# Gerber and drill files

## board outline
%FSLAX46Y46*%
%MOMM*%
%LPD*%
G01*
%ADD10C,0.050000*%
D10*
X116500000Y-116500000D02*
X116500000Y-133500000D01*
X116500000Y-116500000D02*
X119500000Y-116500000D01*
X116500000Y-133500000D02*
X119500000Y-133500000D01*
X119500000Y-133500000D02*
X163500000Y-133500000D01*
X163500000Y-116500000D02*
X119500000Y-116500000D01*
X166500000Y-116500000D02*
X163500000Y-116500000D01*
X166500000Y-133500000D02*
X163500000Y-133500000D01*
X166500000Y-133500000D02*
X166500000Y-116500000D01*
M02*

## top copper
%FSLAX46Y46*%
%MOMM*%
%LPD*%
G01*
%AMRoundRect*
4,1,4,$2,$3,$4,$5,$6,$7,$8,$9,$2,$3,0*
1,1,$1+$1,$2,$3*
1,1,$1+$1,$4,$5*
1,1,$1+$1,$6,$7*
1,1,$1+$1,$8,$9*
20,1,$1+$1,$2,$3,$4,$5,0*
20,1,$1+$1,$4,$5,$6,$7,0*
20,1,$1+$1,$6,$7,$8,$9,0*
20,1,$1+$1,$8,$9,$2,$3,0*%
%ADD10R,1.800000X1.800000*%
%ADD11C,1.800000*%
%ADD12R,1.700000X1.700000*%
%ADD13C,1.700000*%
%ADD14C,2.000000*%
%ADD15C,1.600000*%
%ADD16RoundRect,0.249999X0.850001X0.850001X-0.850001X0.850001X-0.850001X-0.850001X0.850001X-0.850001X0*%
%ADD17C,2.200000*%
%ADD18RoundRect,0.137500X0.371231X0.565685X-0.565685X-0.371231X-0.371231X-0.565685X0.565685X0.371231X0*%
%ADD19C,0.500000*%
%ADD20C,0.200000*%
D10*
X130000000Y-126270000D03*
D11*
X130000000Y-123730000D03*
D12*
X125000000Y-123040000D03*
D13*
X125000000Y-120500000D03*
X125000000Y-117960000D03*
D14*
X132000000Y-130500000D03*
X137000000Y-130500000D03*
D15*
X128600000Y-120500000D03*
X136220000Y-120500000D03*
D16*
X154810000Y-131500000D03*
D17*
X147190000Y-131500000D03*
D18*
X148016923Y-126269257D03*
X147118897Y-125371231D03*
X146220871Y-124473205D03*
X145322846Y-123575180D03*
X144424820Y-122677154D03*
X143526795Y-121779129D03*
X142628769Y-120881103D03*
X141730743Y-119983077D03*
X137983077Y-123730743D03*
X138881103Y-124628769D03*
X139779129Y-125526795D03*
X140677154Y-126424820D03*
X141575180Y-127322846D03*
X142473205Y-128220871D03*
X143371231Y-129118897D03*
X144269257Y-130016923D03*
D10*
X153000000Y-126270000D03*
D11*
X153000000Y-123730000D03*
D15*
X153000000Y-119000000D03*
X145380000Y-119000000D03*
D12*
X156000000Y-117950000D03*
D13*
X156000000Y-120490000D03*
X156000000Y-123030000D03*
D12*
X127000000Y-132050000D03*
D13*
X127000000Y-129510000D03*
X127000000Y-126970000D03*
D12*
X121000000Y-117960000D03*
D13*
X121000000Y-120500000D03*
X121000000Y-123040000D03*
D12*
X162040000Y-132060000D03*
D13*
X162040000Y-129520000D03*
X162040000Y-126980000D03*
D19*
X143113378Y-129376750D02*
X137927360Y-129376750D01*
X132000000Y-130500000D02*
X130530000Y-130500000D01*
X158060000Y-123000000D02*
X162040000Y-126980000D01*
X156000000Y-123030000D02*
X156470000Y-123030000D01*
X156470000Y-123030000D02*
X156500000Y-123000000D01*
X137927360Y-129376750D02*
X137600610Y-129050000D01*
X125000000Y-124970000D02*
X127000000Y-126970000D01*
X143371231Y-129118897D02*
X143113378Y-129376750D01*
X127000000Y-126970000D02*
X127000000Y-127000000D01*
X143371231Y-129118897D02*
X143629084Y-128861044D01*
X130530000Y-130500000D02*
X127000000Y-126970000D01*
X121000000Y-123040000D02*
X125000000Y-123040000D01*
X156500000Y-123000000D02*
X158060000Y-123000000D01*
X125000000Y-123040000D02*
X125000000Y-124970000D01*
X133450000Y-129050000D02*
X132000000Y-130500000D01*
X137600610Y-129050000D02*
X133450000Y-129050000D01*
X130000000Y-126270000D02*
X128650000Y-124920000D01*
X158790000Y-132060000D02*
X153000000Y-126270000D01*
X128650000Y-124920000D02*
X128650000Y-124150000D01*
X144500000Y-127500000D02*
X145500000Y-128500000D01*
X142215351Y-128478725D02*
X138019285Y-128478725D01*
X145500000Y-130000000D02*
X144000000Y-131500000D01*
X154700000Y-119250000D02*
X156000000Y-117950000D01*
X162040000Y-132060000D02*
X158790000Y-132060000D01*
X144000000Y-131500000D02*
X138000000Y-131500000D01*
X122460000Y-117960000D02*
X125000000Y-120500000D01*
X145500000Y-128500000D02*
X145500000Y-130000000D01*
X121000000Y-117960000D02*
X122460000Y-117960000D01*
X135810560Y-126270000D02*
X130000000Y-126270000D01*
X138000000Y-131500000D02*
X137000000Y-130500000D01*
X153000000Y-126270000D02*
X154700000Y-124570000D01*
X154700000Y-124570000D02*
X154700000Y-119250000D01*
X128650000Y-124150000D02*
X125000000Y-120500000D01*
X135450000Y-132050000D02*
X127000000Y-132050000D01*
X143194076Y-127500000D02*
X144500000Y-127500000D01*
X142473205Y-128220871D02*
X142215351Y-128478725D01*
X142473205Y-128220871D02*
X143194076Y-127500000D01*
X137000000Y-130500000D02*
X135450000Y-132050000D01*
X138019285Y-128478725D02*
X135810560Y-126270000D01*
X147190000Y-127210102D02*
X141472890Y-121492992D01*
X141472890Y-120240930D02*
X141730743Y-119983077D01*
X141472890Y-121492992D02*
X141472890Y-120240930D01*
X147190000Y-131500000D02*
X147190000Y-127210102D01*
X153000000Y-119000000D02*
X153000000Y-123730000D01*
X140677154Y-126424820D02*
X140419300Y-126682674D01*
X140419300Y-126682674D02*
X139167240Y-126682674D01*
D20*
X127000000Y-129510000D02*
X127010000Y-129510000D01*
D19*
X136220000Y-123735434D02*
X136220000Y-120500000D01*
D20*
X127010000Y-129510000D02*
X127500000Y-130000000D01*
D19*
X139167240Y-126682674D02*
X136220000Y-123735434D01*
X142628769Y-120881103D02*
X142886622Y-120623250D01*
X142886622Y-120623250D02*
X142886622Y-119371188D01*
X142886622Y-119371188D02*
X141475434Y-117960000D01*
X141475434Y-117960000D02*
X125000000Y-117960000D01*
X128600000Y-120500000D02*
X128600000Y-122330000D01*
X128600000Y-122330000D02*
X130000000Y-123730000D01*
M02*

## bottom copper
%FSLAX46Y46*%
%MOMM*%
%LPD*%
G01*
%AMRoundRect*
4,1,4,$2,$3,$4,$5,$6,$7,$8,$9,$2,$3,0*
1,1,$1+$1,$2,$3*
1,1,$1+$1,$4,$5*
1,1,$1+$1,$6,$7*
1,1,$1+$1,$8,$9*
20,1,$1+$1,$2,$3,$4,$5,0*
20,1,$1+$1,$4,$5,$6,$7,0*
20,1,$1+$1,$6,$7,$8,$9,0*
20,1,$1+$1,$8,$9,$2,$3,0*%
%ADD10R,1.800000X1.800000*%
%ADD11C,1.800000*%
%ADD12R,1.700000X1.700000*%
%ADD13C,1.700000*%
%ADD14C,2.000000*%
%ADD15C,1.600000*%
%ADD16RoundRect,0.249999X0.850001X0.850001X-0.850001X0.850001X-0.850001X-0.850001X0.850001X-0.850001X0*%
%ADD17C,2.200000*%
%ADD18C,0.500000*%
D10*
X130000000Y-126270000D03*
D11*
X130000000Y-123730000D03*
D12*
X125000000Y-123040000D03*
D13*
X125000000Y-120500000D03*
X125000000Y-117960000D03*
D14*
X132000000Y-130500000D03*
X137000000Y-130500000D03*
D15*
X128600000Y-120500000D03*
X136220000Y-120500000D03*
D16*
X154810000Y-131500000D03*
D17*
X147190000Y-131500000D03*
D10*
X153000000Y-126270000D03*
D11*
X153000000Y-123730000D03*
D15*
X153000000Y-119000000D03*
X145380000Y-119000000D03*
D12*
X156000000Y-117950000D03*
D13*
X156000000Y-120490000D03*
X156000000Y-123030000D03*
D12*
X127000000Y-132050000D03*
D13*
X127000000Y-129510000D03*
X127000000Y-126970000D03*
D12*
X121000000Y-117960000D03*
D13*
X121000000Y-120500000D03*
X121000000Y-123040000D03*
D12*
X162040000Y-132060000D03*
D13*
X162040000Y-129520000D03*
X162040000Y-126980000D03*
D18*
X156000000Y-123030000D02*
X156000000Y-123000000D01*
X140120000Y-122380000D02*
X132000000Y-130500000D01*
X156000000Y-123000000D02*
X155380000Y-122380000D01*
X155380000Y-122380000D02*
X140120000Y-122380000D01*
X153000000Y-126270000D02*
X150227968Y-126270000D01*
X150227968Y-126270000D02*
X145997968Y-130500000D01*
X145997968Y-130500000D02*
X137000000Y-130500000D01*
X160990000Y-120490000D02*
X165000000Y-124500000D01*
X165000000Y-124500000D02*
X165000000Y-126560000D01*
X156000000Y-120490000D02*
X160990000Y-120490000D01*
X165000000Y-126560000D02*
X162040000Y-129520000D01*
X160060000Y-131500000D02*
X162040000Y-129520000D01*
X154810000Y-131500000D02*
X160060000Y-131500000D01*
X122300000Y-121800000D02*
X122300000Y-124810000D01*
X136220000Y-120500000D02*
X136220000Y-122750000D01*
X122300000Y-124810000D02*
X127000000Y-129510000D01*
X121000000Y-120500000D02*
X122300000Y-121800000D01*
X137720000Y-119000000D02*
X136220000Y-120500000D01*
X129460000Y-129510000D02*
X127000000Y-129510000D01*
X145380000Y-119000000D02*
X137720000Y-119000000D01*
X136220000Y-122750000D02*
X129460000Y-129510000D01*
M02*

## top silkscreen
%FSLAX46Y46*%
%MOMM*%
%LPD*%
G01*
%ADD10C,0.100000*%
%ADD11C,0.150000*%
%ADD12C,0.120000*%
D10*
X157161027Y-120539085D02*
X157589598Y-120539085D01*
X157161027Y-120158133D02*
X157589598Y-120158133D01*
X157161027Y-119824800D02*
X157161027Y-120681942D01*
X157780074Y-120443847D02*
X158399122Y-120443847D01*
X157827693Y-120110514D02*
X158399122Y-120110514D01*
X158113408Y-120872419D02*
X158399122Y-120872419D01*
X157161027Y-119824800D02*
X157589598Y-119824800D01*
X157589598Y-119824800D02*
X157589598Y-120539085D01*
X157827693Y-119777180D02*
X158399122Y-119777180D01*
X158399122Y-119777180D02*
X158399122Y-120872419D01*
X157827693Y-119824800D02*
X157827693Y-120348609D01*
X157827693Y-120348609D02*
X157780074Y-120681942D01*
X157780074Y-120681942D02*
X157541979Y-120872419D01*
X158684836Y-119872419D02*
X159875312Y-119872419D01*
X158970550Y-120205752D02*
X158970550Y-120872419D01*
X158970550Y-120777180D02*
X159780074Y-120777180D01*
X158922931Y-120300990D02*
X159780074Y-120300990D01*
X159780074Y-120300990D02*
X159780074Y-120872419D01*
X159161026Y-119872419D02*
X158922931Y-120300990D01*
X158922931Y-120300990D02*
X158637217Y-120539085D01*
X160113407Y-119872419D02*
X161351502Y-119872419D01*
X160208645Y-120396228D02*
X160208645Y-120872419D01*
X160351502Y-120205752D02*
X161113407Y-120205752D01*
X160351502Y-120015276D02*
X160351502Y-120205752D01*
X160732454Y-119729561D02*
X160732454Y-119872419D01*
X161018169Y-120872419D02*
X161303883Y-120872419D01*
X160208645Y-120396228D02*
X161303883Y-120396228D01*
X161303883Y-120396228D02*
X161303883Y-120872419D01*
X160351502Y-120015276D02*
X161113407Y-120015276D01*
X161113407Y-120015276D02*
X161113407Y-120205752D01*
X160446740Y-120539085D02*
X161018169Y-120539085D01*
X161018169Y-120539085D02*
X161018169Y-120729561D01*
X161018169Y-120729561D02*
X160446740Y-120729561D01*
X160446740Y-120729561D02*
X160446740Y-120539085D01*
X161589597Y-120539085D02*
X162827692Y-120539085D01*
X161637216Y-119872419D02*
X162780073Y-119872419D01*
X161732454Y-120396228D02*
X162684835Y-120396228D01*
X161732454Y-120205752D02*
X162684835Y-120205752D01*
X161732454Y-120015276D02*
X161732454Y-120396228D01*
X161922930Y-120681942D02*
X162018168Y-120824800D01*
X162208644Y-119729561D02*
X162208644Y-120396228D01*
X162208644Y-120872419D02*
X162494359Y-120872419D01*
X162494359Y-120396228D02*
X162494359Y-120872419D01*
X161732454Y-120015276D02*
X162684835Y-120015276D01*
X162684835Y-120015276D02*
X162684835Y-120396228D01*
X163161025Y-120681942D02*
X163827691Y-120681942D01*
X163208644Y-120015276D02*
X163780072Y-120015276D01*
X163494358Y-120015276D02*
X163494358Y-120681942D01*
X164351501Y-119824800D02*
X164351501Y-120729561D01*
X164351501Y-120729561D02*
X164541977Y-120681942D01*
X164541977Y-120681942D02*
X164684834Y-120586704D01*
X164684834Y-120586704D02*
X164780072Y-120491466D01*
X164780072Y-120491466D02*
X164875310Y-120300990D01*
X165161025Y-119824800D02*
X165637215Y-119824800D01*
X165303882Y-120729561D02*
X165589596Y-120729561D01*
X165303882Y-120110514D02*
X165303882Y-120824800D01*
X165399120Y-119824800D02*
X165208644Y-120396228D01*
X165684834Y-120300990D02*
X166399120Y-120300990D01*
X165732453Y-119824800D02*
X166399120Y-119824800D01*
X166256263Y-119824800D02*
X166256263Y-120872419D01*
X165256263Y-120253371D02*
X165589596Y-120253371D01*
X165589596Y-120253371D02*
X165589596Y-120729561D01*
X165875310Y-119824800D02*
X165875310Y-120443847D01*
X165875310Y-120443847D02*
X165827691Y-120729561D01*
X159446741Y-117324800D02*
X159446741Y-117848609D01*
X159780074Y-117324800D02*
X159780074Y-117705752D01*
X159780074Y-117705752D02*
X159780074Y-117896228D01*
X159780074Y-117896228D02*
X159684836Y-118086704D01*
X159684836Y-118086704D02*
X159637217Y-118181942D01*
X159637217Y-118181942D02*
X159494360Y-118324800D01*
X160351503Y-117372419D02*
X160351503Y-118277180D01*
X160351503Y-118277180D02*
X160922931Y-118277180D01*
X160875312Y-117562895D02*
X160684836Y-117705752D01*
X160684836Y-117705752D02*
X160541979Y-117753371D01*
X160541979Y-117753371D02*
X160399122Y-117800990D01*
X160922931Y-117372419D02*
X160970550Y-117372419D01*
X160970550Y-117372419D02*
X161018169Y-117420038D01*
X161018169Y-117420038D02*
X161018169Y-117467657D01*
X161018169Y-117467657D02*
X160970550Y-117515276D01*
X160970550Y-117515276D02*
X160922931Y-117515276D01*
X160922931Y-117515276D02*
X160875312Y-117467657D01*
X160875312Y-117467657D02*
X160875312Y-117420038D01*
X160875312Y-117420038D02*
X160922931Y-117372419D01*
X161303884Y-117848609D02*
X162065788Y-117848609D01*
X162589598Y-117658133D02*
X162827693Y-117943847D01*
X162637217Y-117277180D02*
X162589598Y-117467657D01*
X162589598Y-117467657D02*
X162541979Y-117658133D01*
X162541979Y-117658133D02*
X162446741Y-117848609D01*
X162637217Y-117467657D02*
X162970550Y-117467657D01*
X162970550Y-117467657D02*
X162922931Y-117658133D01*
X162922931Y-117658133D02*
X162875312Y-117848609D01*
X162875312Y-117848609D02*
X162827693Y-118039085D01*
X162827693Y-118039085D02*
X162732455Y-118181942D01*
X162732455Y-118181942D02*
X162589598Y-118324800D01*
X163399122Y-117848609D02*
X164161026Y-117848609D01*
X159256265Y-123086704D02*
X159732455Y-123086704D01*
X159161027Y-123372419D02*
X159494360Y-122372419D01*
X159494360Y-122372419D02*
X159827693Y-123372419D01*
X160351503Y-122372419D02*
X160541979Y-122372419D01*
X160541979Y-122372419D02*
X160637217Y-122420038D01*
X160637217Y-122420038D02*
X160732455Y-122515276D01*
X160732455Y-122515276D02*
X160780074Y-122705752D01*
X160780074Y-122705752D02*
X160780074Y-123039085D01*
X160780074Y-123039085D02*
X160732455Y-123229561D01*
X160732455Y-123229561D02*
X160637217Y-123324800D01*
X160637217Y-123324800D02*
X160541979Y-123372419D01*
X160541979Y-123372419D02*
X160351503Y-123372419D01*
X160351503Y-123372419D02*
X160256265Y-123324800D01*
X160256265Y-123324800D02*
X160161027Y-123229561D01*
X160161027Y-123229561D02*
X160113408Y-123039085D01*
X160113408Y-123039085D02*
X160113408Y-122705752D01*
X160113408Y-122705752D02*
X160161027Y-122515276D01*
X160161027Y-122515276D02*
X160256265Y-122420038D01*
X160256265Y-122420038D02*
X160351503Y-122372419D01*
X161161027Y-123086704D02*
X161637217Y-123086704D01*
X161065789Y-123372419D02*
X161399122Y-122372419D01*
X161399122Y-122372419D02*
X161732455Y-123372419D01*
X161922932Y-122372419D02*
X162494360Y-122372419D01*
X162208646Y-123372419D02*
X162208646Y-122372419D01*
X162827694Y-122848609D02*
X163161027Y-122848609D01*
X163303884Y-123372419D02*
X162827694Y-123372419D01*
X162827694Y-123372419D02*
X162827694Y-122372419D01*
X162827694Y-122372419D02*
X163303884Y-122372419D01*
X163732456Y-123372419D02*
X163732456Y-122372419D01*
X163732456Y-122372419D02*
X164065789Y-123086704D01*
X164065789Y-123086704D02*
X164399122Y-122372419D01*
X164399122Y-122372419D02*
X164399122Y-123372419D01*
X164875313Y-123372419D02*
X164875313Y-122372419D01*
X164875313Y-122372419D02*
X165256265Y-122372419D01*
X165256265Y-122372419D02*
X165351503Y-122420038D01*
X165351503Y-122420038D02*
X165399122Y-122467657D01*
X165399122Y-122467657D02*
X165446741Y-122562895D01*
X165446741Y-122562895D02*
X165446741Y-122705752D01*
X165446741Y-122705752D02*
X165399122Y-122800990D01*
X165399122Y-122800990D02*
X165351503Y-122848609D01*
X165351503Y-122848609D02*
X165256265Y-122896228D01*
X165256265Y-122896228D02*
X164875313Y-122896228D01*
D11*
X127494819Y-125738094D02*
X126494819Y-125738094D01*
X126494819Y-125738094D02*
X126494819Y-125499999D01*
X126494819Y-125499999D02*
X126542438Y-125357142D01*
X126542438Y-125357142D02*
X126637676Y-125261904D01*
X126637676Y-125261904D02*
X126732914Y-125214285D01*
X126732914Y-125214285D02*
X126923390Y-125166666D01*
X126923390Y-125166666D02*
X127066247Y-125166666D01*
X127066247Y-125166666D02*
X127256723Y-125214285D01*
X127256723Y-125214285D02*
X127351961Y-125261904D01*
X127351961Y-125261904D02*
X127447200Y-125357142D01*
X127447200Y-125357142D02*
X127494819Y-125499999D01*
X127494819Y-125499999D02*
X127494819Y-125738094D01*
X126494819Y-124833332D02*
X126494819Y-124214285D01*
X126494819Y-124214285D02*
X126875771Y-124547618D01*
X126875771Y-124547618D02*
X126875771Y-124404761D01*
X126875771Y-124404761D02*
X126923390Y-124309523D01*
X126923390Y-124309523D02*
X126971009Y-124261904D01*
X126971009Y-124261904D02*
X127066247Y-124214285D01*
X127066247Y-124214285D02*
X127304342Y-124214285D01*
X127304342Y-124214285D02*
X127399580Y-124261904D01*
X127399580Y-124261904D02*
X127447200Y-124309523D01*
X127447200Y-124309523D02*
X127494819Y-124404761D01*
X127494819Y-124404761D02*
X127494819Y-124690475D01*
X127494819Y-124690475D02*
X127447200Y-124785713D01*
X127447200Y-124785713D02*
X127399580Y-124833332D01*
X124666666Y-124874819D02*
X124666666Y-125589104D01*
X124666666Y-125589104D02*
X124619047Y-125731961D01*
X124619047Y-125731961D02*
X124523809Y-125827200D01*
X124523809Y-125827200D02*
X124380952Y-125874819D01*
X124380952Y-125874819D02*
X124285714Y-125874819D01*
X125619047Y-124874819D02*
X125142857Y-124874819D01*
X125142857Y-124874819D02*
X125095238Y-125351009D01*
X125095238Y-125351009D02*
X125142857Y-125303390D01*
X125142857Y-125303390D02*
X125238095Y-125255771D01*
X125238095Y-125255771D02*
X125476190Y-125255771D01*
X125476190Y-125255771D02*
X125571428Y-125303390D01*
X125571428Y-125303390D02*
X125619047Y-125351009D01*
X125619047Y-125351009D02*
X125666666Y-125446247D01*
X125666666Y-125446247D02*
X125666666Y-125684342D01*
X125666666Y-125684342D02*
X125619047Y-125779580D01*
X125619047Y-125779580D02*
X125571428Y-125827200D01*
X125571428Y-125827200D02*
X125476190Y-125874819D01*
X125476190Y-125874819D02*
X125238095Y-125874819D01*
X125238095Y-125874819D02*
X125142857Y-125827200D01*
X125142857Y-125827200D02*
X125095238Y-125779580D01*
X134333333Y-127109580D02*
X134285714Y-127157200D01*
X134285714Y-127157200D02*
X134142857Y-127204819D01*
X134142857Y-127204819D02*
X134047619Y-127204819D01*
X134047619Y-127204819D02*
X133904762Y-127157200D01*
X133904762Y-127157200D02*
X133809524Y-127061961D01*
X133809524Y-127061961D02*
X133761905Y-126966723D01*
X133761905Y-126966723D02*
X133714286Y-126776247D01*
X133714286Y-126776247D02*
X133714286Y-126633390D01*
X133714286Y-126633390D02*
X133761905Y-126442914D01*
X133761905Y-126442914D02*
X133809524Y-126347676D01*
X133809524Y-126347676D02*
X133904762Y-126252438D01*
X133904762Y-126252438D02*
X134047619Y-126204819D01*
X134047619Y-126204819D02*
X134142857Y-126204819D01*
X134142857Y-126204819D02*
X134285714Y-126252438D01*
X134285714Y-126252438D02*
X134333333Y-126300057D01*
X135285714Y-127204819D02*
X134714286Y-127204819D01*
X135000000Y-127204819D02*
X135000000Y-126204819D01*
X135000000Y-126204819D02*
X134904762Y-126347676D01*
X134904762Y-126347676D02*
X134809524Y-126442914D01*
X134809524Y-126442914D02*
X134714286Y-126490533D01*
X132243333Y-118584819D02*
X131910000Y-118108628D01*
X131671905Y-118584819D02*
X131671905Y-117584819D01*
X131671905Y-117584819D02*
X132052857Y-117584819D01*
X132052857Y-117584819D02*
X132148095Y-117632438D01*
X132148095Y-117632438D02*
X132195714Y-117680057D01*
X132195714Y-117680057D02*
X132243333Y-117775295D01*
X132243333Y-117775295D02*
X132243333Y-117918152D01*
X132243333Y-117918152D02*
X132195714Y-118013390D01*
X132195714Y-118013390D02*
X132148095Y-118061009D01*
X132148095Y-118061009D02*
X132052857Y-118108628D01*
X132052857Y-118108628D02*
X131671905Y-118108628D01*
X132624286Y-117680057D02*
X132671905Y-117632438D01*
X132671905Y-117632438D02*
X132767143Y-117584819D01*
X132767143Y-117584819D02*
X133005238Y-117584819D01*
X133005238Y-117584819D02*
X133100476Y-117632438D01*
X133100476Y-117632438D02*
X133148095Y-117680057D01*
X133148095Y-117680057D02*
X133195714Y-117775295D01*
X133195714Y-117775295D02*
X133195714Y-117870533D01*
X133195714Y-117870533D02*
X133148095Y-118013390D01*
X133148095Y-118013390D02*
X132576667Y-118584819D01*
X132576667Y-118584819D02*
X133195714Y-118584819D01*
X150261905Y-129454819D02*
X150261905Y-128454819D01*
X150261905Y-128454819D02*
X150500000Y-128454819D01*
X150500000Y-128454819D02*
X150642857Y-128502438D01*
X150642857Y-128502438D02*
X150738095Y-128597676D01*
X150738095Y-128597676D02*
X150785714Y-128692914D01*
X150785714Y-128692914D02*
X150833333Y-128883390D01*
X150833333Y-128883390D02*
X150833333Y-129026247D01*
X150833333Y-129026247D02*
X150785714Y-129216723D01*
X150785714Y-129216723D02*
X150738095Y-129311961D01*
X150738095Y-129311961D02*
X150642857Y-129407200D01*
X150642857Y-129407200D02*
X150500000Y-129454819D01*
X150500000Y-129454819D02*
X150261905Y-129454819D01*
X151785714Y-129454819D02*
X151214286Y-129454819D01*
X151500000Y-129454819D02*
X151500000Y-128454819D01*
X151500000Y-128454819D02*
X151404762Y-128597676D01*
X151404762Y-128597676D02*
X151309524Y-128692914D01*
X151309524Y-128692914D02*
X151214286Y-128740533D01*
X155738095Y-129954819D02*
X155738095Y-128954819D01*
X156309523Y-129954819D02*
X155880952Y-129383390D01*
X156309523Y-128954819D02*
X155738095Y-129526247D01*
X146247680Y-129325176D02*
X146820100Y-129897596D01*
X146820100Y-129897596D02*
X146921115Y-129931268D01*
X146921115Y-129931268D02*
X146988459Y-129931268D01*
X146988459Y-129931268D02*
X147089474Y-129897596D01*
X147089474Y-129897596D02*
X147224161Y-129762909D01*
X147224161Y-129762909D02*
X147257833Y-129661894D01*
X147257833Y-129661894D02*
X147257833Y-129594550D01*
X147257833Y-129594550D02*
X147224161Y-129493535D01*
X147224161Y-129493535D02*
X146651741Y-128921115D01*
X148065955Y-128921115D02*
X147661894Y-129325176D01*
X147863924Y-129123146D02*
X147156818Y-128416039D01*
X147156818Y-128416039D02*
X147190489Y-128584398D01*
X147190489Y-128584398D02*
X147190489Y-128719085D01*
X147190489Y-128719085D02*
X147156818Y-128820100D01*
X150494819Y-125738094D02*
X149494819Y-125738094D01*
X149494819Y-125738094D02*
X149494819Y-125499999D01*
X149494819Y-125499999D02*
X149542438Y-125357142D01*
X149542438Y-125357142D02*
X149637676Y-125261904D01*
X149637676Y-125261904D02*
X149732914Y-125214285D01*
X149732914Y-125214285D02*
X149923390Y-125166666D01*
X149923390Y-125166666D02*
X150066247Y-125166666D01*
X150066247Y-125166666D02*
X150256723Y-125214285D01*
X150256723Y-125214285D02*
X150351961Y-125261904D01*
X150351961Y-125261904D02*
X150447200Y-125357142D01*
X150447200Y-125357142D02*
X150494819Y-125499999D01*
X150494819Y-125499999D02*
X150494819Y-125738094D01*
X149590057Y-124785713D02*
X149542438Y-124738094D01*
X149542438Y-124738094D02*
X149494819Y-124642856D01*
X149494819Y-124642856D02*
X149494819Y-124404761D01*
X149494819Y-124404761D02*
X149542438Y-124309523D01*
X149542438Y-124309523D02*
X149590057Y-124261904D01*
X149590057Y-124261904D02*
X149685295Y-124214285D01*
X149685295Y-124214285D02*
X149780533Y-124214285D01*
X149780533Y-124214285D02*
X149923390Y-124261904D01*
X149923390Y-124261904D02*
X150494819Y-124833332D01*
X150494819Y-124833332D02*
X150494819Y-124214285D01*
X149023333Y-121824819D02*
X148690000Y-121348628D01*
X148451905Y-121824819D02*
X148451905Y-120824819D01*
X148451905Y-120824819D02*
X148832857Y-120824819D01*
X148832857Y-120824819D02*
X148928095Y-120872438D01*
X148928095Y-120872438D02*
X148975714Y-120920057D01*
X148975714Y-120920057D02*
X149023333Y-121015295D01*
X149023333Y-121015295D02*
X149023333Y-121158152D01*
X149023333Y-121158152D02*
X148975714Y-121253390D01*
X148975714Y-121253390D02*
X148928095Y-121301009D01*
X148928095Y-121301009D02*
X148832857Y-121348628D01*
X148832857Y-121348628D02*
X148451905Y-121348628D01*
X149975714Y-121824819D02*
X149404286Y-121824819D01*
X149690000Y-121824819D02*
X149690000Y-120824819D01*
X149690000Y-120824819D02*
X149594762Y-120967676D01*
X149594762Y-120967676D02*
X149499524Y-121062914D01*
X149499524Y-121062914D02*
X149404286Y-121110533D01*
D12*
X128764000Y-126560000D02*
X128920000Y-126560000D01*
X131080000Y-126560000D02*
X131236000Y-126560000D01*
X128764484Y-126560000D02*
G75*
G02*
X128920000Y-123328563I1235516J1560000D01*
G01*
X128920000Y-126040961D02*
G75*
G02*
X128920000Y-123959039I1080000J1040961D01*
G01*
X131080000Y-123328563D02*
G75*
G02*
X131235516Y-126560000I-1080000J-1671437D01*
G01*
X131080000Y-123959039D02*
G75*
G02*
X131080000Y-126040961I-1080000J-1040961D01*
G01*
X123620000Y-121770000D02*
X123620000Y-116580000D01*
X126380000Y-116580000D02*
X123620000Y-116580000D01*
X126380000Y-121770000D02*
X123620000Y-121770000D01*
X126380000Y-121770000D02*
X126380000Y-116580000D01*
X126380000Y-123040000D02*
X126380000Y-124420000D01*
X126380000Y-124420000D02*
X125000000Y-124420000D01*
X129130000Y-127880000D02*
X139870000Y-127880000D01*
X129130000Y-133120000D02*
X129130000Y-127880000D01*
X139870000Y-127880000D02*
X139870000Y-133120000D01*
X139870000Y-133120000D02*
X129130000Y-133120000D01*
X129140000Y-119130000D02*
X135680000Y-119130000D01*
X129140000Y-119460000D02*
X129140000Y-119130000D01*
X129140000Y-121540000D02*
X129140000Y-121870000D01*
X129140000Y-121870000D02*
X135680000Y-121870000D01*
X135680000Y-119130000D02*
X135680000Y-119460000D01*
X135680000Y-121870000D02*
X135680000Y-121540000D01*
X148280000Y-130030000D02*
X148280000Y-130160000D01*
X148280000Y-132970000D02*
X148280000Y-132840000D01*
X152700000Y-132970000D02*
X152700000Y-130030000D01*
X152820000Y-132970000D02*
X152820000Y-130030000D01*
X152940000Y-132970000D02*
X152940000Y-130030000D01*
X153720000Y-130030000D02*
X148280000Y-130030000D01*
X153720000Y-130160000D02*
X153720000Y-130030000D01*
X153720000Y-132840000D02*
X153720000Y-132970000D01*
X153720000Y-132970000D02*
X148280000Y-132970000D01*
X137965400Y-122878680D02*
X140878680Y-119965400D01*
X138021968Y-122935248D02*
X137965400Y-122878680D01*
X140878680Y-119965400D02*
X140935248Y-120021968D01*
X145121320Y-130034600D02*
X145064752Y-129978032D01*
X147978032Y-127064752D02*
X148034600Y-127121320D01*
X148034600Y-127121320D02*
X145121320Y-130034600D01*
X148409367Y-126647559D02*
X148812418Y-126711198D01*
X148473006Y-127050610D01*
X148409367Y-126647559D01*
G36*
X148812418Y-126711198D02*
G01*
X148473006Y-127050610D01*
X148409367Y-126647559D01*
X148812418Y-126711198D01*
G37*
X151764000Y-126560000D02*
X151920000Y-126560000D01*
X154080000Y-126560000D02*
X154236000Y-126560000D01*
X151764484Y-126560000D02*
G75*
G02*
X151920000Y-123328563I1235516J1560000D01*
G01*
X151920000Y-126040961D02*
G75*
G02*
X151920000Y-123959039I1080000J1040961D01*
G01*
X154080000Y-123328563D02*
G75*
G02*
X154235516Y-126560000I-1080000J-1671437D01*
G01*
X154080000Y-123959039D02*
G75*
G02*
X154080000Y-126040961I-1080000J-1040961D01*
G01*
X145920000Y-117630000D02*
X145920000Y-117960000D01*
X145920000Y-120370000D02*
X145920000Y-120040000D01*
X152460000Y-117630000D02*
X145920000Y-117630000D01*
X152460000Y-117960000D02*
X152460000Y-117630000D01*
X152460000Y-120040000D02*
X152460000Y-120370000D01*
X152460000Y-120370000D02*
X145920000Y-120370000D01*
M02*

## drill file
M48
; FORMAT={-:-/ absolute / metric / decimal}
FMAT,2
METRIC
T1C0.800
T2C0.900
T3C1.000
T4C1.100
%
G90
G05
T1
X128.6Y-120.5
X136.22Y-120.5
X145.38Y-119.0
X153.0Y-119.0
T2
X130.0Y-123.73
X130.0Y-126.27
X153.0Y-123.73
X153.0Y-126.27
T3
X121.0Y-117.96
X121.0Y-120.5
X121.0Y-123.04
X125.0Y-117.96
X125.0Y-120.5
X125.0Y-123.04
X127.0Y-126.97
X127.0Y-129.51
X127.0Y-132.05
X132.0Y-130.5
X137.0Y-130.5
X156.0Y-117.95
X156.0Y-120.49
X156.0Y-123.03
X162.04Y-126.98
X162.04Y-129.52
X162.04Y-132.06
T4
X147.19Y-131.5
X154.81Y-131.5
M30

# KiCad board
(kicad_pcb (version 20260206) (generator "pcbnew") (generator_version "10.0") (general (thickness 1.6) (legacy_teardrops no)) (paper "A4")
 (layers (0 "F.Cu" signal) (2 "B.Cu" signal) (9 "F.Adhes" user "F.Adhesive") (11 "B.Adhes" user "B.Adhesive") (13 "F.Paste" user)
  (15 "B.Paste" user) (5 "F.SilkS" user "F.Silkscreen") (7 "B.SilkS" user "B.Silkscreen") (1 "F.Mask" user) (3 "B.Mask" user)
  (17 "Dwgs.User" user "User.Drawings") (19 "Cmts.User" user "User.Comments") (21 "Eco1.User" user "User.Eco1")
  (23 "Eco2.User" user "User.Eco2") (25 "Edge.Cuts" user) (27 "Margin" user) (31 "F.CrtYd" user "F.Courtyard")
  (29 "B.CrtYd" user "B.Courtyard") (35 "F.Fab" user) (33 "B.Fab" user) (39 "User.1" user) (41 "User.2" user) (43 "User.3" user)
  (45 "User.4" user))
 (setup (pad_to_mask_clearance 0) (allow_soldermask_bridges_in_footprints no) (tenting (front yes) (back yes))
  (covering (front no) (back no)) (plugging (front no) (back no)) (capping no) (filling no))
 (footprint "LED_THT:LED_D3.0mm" (layer "F.Cu") (at 130 126.27 90)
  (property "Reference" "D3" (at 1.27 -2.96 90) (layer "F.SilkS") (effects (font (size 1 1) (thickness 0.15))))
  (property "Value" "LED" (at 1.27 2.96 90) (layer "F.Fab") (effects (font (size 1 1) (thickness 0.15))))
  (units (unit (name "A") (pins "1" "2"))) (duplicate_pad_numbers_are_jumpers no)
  (fp_line (start -0.29 -1.236) (end -0.29 -1.08) (stroke (width 0.12) (type solid)) (layer "F.SilkS"))
  (fp_line (start -0.29 1.08) (end -0.29 1.236) (stroke (width 0.12) (type solid)) (layer "F.SilkS"))
  (fp_arc (start -0.29 -1.235516) (mid 1.36566 -1.987699) (end 2.941437 -1.08) (stroke (width 0.12) (type solid)) (layer "F.SilkS"))
  (fp_arc (start 0.229039 -1.08) (mid 1.27 -1.5) (end 2.310961 -1.08) (stroke (width 0.12) (type solid)) (layer "F.SilkS"))
  (fp_arc (start 2.941437 1.08) (mid 1.36566 1.987699) (end -0.29 1.235516) (stroke (width 0.12) (type solid)) (layer "F.SilkS"))
  (fp_arc (start 2.310961 1.08) (mid 1.27 1.5) (end 0.229039 1.08) (stroke (width 0.12) (type solid)) (layer "F.SilkS"))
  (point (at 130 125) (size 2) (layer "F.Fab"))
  (pad "1" thru_hole rect (at 0 0 90) (size 1.8 1.8) (drill 0.9) (layers "*.Cu" "*.Mask") (remove_unused_layers no) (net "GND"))
  (pad "2" thru_hole circle (at 2.54 0 90) (size 1.8 1.8) (drill 0.9) (layers "*.Cu" "*.Mask") (remove_unused_layers no) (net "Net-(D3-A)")))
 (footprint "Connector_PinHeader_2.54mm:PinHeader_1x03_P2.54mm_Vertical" (layer "F.Cu") (at 125 123.04 180)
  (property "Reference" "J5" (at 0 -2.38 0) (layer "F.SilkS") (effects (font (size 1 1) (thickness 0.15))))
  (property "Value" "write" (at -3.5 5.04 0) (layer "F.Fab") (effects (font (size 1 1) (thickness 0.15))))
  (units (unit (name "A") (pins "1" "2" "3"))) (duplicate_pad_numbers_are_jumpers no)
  (fp_line (start 1.38 1.27) (end 1.38 6.46) (stroke (width 0.12) (type solid)) (layer "F.SilkS"))
  (fp_line (start -1.38 6.46) (end 1.38 6.46) (stroke (width 0.12) (type solid)) (layer "F.SilkS"))
  (fp_line (start -1.38 1.27) (end 1.38 1.27) (stroke (width 0.12) (type solid)) (layer "F.SilkS"))
  (fp_line (start -1.38 1.27) (end -1.38 6.46) (stroke (width 0.12) (type solid)) (layer "F.SilkS"))
  (fp_line (start -1.38 0) (end -1.38 -1.38) (stroke (width 0.12) (type solid)) (layer "F.SilkS"))
  (fp_line (start -1.38 -1.38) (end 0 -1.38) (stroke (width 0.12) (type solid)) (layer "F.SilkS"))
  (pad "1" thru_hole rect (at 0 0 180) (size 1.7 1.7) (drill 1) (layers "*.Cu" "*.Mask") (remove_unused_layers no) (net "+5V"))
  (pad "2" thru_hole circle (at 0 2.54 180) (size 1.7 1.7) (drill 1) (layers "*.Cu" "*.Mask") (remove_unused_layers no) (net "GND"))
  (pad "3" thru_hole circle (at 0 5.08 180) (size 1.7 1.7) (drill 1) (layers "*.Cu" "*.Mask") (remove_unused_layers no) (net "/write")))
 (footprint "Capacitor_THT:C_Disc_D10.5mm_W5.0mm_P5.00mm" (layer "F.Cu") (at 132 130.5)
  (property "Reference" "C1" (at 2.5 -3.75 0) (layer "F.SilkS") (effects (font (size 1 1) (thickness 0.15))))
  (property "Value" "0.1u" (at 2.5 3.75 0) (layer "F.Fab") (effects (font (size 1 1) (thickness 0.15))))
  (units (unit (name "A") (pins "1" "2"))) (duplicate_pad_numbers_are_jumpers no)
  (fp_line (start -2.87 -2.62) (end 7.87 -2.62) (stroke (width 0.12) (type solid)) (layer "F.SilkS"))
  (fp_line (start -2.87 2.62) (end -2.87 -2.62) (stroke (width 0.12) (type solid)) (layer "F.SilkS"))
  (fp_line (start 7.87 -2.62) (end 7.87 2.62) (stroke (width 0.12) (type solid)) (layer "F.SilkS"))
  (fp_line (start 7.87 2.62) (end -2.87 2.62) (stroke (width 0.12) (type solid)) (layer "F.SilkS"))
  (pad "1" thru_hole circle (at 0 0) (size 2 2) (drill 1) (layers "*.Cu" "*.Mask") (remove_unused_layers no) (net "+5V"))
  (pad "2" thru_hole circle (at 5 0) (size 2 2) (drill 1) (layers "*.Cu" "*.Mask") (remove_unused_layers no) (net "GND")))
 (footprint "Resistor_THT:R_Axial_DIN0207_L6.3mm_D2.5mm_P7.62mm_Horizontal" (layer "F.Cu") (at 128.6 120.5)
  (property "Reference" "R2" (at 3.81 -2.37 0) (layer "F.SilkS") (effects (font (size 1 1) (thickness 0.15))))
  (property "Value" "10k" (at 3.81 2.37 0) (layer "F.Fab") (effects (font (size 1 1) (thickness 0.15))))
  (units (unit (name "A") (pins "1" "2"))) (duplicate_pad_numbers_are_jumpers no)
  (fp_line (start 0.54 -1.37) (end 7.08 -1.37) (stroke (width 0.12) (type solid)) (layer "F.SilkS"))
  (fp_line (start 0.54 -1.04) (end 0.54 -1.37) (stroke (width 0.12) (type solid)) (layer "F.SilkS"))
  (fp_line (start 0.54 1.04) (end 0.54 1.37) (stroke (width 0.12) (type solid)) (layer "F.SilkS"))
  (fp_line (start 0.54 1.37) (end 7.08 1.37) (stroke (width 0.12) (type solid)) (layer "F.SilkS"))
  (fp_line (start 7.08 -1.37) (end 7.08 -1.04) (stroke (width 0.12) (type solid)) (layer "F.SilkS"))
  (fp_line (start 7.08 1.37) (end 7.08 1.04) (stroke (width 0.12) (type solid)) (layer "F.SilkS"))
  (pad "1" thru_hole circle (at 0 0) (size 1.6 1.6) (drill 0.8) (layers "*.Cu" "*.Mask") (remove_unused_layers no) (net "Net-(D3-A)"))
  (pad "2" thru_hole circle (at 7.62 0) (size 1.6 1.6) (drill 0.8) (layers "*.Cu" "*.Mask") (remove_unused_layers no) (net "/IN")))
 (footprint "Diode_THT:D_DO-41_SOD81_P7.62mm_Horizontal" (layer "F.Cu") (at 154.81 131.5 180)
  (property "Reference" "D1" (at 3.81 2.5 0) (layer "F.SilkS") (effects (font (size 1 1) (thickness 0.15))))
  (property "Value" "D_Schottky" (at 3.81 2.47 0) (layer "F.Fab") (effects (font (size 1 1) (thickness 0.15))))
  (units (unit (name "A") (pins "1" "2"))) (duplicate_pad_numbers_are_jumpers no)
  (fp_line (start 6.53 1.47) (end 6.53 1.34) (stroke (width 0.12) (type solid)) (layer "F.SilkS"))
  (fp_line (start 6.53 -1.47) (end 6.53 -1.34) (stroke (width 0.12) (type solid)) (layer "F.SilkS"))
  (fp_line (start 2.11 -1.47) (end 2.11 1.47) (stroke (width 0.12) (type solid)) (layer "F.SilkS"))
  (fp_line (start 1.99 -1.47) (end 1.99 1.47) (stroke (width 0.12) (type solid)) (layer "F.SilkS"))
  (fp_line (start 1.87 -1.47) (end 1.87 1.47) (stroke (width 0.12) (type solid)) (layer "F.SilkS"))
  (fp_line (start 1.09 1.47) (end 6.53 1.47) (stroke (width 0.12) (type solid)) (layer "F.SilkS"))
  (fp_line (start 1.09 1.34) (end 1.09 1.47) (stroke (width 0.12) (type solid)) (layer "F.SilkS"))
  (fp_line (start 1.09 -1.34) (end 1.09 -1.47) (stroke (width 0.12) (type solid)) (layer "F.SilkS"))
  (fp_line (start 1.09 -1.47) (end 6.53 -1.47) (stroke (width 0.12) (type solid)) (layer "F.SilkS"))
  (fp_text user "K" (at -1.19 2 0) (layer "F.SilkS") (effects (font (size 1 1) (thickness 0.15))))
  (pad "1" thru_hole roundrect (at 0 0 180) (size 2.2 2.2) (drill 1.1) (layers "*.Cu" "*.Mask") (remove_unused_layers no)
   (roundrect_rratio 0.113636) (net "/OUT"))
  (pad "2" thru_hole circle (at 7.62 0 180) (size 2.2 2.2) (drill 1.1) (layers "*.Cu" "*.Mask") (remove_unused_layers no) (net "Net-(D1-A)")))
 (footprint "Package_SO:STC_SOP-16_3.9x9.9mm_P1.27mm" (layer "F.Cu") (at 143 125 -135)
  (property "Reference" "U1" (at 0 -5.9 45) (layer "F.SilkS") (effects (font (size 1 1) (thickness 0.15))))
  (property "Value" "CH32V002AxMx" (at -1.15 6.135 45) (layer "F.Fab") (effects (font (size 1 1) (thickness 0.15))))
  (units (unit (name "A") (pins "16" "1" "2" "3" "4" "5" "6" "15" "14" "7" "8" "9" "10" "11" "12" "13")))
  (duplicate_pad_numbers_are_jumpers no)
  (fp_line (start 2.06 5.06) (end -2.06 5.06) (stroke (width 0.12) (type solid)) (layer "F.SilkS"))
  (fp_line (start 2.06 4.98) (end 2.06 5.06) (stroke (width 0.12) (type solid)) (layer "F.SilkS"))
  (fp_line (start -2.06 5.06) (end -2.06 4.98) (stroke (width 0.12) (type solid)) (layer "F.SilkS"))
  (fp_line (start 2.06 -5.06) (end 2.06 -4.98) (stroke (width 0.12) (type solid)) (layer "F.SilkS"))
  (fp_line (start -2.06 -4.98) (end -2.06 -5.06) (stroke (width 0.12) (type solid)) (layer "F.SilkS"))
  (fp_line (start -2.06 -5.06) (end 2.06 -5.06) (stroke (width 0.12) (type solid)) (layer "F.SilkS"))
  (fp_poly (pts (xy -2.66 -4.99) (xy -2.9 -5.32) (xy -2.419999 -5.32)) (stroke (width 0.12) (type solid)) (fill yes) (layer "F.SilkS"))
  (pad "1" smd roundrect (at -2.65 -4.445001 225) (size 1.6 0.55) (layers "F.Cu" "F.Mask" "F.Paste") (roundrect_rratio 0.25)
   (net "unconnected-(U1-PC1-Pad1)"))
  (pad "2" smd roundrect (at -2.65 -3.175 225) (size 1.6 0.55) (layers "F.Cu" "F.Mask" "F.Paste") (roundrect_rratio 0.25)
   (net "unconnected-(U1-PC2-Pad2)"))
  (pad "3" smd roundrect (at -2.65 -1.904999 225) (size 1.6 0.55) (layers "F.Cu" "F.Mask" "F.Paste") (roundrect_rratio 0.25)
   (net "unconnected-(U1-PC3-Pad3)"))
  (pad "4" smd roundrect (at -2.65 -0.635 225) (size 1.6 0.55) (layers "F.Cu" "F.Mask" "F.Paste") (roundrect_rratio 0.25)
   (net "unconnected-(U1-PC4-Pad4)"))
  (pad "5" smd roundrect (at -2.65 0.635 225) (size 1.6 0.55) (layers "F.Cu" "F.Mask" "F.Paste") (roundrect_rratio 0.25)
   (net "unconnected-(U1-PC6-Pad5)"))
  (pad "6" smd roundrect (at -2.65 1.904999 225) (size 1.6 0.55) (layers "F.Cu" "F.Mask" "F.Paste") (roundrect_rratio 0.25)
   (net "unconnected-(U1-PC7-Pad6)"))
  (pad "7" smd roundrect (at -2.65 3.175 225) (size 1.6 0.55) (layers "F.Cu" "F.Mask" "F.Paste") (roundrect_rratio 0.25) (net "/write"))
  (pad "8" smd roundrect (at -2.65 4.445001 225) (size 1.6 0.55) (layers "F.Cu" "F.Mask" "F.Paste") (roundrect_rratio 0.25)
   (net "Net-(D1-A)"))
  (pad "9" smd roundrect (at 2.65 4.445001 225) (size 1.6 0.55) (layers "F.Cu" "F.Mask" "F.Paste") (roundrect_rratio 0.25)
   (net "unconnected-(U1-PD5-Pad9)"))
  (pad "10" smd roundrect (at 2.65 3.175 225) (size 1.6 0.55) (layers "F.Cu" "F.Mask" "F.Paste") (roundrect_rratio 0.25)
   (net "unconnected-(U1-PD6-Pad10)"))
  (pad "11" smd roundrect (at 2.65 1.904999 225) (size 1.6 0.55) (layers "F.Cu" "F.Mask" "F.Paste") (roundrect_rratio 0.25)
   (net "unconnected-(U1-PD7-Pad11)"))
  (pad "12" smd roundrect (at 2.65 0.635 225) (size 1.6 0.55) (layers "F.Cu" "F.Mask" "F.Paste") (roundrect_rratio 0.25) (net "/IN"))
  (pad "13" smd roundrect (at 2.65 -0.635 225) (size 1.6 0.55) (layers "F.Cu" "F.Mask" "F.Paste") (roundrect_rratio 0.25)
   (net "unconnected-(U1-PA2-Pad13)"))
  (pad "14" smd roundrect (at 2.65 -1.904999 225) (size 1.6 0.55) (layers "F.Cu" "F.Mask" "F.Paste") (roundrect_rratio 0.25) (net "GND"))
  (pad "15" smd roundrect (at 2.65 -3.175 225) (size 1.6 0.55) (layers "F.Cu" "F.Mask" "F.Paste") (roundrect_rratio 0.25) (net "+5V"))
  (pad "16" smd roundrect (at 2.65 -4.445001 225) (size 1.6 0.55) (layers "F.Cu" "F.Mask" "F.Paste") (roundrect_rratio 0.25)
   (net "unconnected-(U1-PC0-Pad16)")))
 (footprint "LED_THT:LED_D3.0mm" (layer "F.Cu") (at 153 126.27 90)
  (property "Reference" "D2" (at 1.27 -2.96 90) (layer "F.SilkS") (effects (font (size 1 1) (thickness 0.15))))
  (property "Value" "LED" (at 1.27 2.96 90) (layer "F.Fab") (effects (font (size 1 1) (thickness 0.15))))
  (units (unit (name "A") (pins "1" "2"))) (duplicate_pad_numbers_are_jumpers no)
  (fp_line (start -0.29 -1.236) (end -0.29 -1.08) (stroke (width 0.12) (type solid)) (layer "F.SilkS"))
  (fp_line (start -0.29 1.08) (end -0.29 1.236) (stroke (width 0.12) (type solid)) (layer "F.SilkS"))
  (fp_arc (start -0.29 -1.235516) (mid 1.36566 -1.987699) (end 2.941437 -1.08) (stroke (width 0.12) (type solid)) (layer "F.SilkS"))
  (fp_arc (start 0.229039 -1.08) (mid 1.27 -1.5) (end 2.310961 -1.08) (stroke (width 0.12) (type solid)) (layer "F.SilkS"))
  (fp_arc (start 2.941437 1.08) (mid 1.36566 1.987699) (end -0.29 1.235516) (stroke (width 0.12) (type solid)) (layer "F.SilkS"))
  (fp_arc (start 2.310961 1.08) (mid 1.27 1.5) (end 0.229039 1.08) (stroke (width 0.12) (type solid)) (layer "F.SilkS"))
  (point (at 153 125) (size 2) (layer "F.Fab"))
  (pad "1" thru_hole rect (at 0 0 90) (size 1.8 1.8) (drill 0.9) (layers "*.Cu" "*.Mask") (remove_unused_layers no) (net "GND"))
  (pad "2" thru_hole circle (at 2.54 0 90) (size 1.8 1.8) (drill 0.9) (layers "*.Cu" "*.Mask") (remove_unused_layers no) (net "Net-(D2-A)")))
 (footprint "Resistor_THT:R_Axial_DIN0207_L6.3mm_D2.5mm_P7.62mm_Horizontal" (layer "F.Cu") (at 153 119 180)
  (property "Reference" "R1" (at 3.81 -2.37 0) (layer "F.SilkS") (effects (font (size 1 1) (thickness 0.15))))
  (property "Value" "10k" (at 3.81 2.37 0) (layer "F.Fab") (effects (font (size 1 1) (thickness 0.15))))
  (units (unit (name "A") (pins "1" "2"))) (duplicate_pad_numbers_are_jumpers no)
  (fp_line (start 7.08 1.37) (end 7.08 1.04) (stroke (width 0.12) (type solid)) (layer "F.SilkS"))
  (fp_line (start 7.08 -1.37) (end 7.08 -1.04) (stroke (width 0.12) (type solid)) (layer "F.SilkS"))
  (fp_line (start 0.54 1.37) (end 7.08 1.37) (stroke (width 0.12) (type solid)) (layer "F.SilkS"))
  (fp_line (start 0.54 1.04) (end 0.54 1.37) (stroke (width 0.12) (type solid)) (layer "F.SilkS"))
  (fp_line (start 0.54 -1.04) (end 0.54 -1.37) (stroke (width 0.12) (type solid)) (layer "F.SilkS"))
  (fp_line (start 0.54 -1.37) (end 7.08 -1.37) (stroke (width 0.12) (type solid)) (layer "F.SilkS"))
  (pad "1" thru_hole circle (at 0 0 180) (size 1.6 1.6) (drill 0.8) (layers "*.Cu" "*.Mask") (remove_unused_layers no) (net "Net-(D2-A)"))
  (pad "2" thru_hole circle (at 7.62 0 180) (size 1.6 1.6) (drill 0.8) (layers "*.Cu" "*.Mask") (remove_unused_layers no) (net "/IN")))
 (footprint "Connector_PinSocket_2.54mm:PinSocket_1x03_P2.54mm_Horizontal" (layer "B.Cu") (at 156 117.95 180)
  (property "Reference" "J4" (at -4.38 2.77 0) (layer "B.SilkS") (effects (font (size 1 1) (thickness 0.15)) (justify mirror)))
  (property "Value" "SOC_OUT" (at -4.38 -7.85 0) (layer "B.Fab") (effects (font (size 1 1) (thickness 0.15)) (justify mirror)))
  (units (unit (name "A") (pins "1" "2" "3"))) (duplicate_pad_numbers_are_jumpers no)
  (pad "1" thru_hole rect (at 0 0 180) (size 1.7 1.7) (drill 1) (layers "*.Cu" "*.Mask") (remove_unused_layers no) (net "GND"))
  (pad "2" thru_hole circle (at 0 -2.54 180) (size 1.7 1.7) (drill 1) (layers "*.Cu" "*.Mask") (remove_unused_layers no) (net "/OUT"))
  (pad "3" thru_hole circle (at 0 -5.08 180) (size 1.7 1.7) (drill 1) (layers "*.Cu" "*.Mask") (remove_unused_layers no) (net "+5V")))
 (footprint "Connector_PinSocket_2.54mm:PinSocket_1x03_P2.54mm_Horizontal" (layer "B.Cu") (at 127 132.05)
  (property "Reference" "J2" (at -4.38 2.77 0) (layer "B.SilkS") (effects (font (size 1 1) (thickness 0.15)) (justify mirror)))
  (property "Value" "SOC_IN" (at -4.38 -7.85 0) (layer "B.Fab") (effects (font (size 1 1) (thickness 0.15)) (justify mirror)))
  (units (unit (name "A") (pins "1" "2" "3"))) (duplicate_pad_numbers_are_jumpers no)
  (pad "1" thru_hole rect (at 0 0) (size 1.7 1.7) (drill 1) (layers "*.Cu" "*.Mask") (remove_unused_layers no) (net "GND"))
  (pad "2" thru_hole circle (at 0 -2.54) (size 1.7 1.7) (drill 1) (layers "*.Cu" "*.Mask") (remove_unused_layers no) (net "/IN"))
  (pad "3" thru_hole circle (at 0 -5.08) (size 1.7 1.7) (drill 1) (layers "*.Cu" "*.Mask") (remove_unused_layers no) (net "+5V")))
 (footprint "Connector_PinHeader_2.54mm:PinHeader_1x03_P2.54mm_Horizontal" (layer "B.Cu") (at 121 117.96 180)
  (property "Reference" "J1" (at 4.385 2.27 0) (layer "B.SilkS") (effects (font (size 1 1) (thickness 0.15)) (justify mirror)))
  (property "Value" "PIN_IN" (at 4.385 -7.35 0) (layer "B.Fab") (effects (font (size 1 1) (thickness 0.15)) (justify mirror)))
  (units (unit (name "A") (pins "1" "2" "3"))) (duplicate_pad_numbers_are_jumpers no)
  (pad "1" thru_hole rect (at 0 0 180) (size 1.7 1.7) (drill 1) (layers "*.Cu" "*.Mask") (remove_unused_layers no) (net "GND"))
  (pad "2" thru_hole circle (at 0 -2.54 180) (size 1.7 1.7) (drill 1) (layers "*.Cu" "*.Mask") (remove_unused_layers no) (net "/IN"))
  (pad "3" thru_hole circle (at 0 -5.08 180) (size 1.7 1.7) (drill 1) (layers "*.Cu" "*.Mask") (remove_unused_layers no) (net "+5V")))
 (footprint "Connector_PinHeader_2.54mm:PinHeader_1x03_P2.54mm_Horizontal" (layer "B.Cu") (at 162.04 132.06)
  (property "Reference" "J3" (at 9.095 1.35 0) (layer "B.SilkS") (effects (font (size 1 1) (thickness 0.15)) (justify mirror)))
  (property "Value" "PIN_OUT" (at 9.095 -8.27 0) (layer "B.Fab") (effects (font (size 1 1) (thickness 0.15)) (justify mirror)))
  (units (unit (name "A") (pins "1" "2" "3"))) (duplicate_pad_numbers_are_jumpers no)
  (pad "1" thru_hole rect (at 0 0) (size 1.7 1.7) (drill 1) (layers "*.Cu" "*.Mask") (remove_unused_layers no) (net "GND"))
  (pad "2" thru_hole circle (at 0 -2.54) (size 1.7 1.7) (drill 1) (layers "*.Cu" "*.Mask") (remove_unused_layers no) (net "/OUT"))
  (pad "3" thru_hole circle (at 0 -5.08) (size 1.7 1.7) (drill 1) (layers "*.Cu" "*.Mask") (remove_unused_layers no) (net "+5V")))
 (gr_line (start 116.5 116.5) (end 116.5 133.5) (stroke (width 0.05) (type default)) (layer "Edge.Cuts"))
 (gr_line (start 116.5 116.5) (end 119.5 116.5) (stroke (width 0.05) (type default)) (layer "Edge.Cuts"))
 (gr_line (start 116.5 133.5) (end 119.5 133.5) (stroke (width 0.05) (type default)) (layer "Edge.Cuts"))
 (gr_line (start 119.5 133.5) (end 163.5 133.5) (stroke (width 0.05) (type default)) (layer "Edge.Cuts"))
 (gr_line (start 163.5 116.5) (end 119.5 116.5) (stroke (width 0.05) (type default)) (layer "Edge.Cuts"))
 (gr_line (start 166.5 116.5) (end 163.5 116.5) (stroke (width 0.05) (type default)) (layer "Edge.Cuts"))
 (gr_line (start 166.5 133.5) (end 163.5 133.5) (stroke (width 0.05) (type default)) (layer "Edge.Cuts"))
 (gr_line (start 166.5 133.5) (end 166.5 116.5) (stroke (width 0.05) (type default)) (layer "Edge.Cuts"))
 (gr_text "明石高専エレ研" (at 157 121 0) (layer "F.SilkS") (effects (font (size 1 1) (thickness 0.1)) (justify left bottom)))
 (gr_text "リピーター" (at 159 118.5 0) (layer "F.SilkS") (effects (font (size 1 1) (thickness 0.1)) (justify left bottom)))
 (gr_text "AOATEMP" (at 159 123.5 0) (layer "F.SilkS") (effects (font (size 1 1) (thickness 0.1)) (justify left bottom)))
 (segment (start 143.113378 129.37675) (end 137.92736 129.37675) (width 0.5) (layer "F.Cu") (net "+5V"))
 (segment (start 132 130.5) (end 130.53 130.5) (width 0.5) (layer "F.Cu") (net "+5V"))
 (segment (start 158.06 123) (end 162.04 126.98) (width 0.5) (layer "F.Cu") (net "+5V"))
 (segment (start 156 123.03) (end 156.47 123.03) (width 0.5) (layer "F.Cu") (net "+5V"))
 (segment (start 156.47 123.03) (end 156.5 123) (width 0.5) (layer "F.Cu") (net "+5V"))
 (segment (start 137.92736 129.37675) (end 137.60061 129.05) (width 0.5) (layer "F.Cu") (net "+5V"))
 (segment (start 125 124.97) (end 127 126.97) (width 0.5) (layer "F.Cu") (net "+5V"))
 (segment (start 143.371231 129.118897) (end 143.113378 129.37675) (width 0.5) (layer "F.Cu") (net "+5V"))
 (segment (start 127 126.97) (end 127 127) (width 0.5) (layer "F.Cu") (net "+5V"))
 (segment (start 143.371231 129.118897) (end 143.629084 128.861044) (width 0.5) (layer "F.Cu") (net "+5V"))
 (segment (start 130.53 130.5) (end 127 126.97) (width 0.5) (layer "F.Cu") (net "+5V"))
 (segment (start 121 123.04) (end 125 123.04) (width 0.5) (layer "F.Cu") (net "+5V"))
 (segment (start 156.5 123) (end 158.06 123) (width 0.5) (layer "F.Cu") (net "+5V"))
 (segment (start 125 123.04) (end 125 124.97) (width 0.5) (layer "F.Cu") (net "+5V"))
 (segment (start 133.45 129.05) (end 132 130.5) (width 0.5) (layer "F.Cu") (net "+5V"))
 (segment (start 137.60061 129.05) (end 133.45 129.05) (width 0.5) (layer "F.Cu") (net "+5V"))
 (segment (start 156 123.03) (end 156 123) (width 0.5) (layer "B.Cu") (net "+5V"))
 (segment (start 140.12 122.38) (end 132 130.5) (width 0.5) (layer "B.Cu") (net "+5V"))
 (segment (start 156 123) (end 155.38 122.38) (width 0.5) (layer "B.Cu") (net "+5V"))
 (segment (start 155.38 122.38) (end 140.12 122.38) (width 0.5) (layer "B.Cu") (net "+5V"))
 (segment (start 130 126.27) (end 128.65 124.92) (width 0.5) (layer "F.Cu") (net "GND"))
 (segment (start 158.79 132.06) (end 153 126.27) (width 0.5) (layer "F.Cu") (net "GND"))
 (segment (start 128.65 124.92) (end 128.65 124.15) (width 0.5) (layer "F.Cu") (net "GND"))
 (segment (start 144.5 127.5) (end 145.5 128.5) (width 0.5) (layer "F.Cu") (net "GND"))
 (segment (start 142.215351 128.478725) (end 138.019285 128.478725) (width 0.5) (layer "F.Cu") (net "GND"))
 (segment (start 145.5 130) (end 144 131.5) (width 0.5) (layer "F.Cu") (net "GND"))
 (segment (start 154.7 119.25) (end 156 117.95) (width 0.5) (layer "F.Cu") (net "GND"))
 (segment (start 162.04 132.06) (end 158.79 132.06) (width 0.5) (layer "F.Cu") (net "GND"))
 (segment (start 144 131.5) (end 138 131.5) (width 0.5) (layer "F.Cu") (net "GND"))
 (segment (start 122.46 117.96) (end 125 120.5) (width 0.5) (layer "F.Cu") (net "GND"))
 (segment (start 145.5 128.5) (end 145.5 130) (width 0.5) (layer "F.Cu") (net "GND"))
 (segment (start 121 117.96) (end 122.46 117.96) (width 0.5) (layer "F.Cu") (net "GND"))
 (segment (start 135.81056 126.27) (end 130 126.27) (width 0.5) (layer "F.Cu") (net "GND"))
 (segment (start 138 131.5) (end 137 130.5) (width 0.5) (layer "F.Cu") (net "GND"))
 (segment (start 153 126.27) (end 154.7 124.57) (width 0.5) (layer "F.Cu") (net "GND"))
 (segment (start 154.7 124.57) (end 154.7 119.25) (width 0.5) (layer "F.Cu") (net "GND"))
 (segment (start 128.65 124.15) (end 125 120.5) (width 0.5) (layer "F.Cu") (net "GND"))
 (segment (start 135.45 132.05) (end 127 132.05) (width 0.5) (layer "F.Cu") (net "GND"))
 (segment (start 143.194076 127.5) (end 144.5 127.5) (width 0.5) (layer "F.Cu") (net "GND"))
 (segment (start 142.473205 128.220871) (end 142.215351 128.478725) (width 0.5) (layer "F.Cu") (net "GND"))
 (segment (start 142.473205 128.220871) (end 143.194076 127.5) (width 0.5) (layer "F.Cu") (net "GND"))
 (segment (start 137 130.5) (end 135.45 132.05) (width 0.5) (layer "F.Cu") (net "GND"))
 (segment (start 138.019285 128.478725) (end 135.81056 126.27) (width 0.5) (layer "F.Cu") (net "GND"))
 (segment (start 153 126.27) (end 150.227968 126.27) (width 0.5) (layer "B.Cu") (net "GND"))
 (segment (start 150.227968 126.27) (end 145.997968 130.5) (width 0.5) (layer "B.Cu") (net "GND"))
 (segment (start 145.997968 130.5) (end 137 130.5) (width 0.5) (layer "B.Cu") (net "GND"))
 (segment (start 147.19 127.210102) (end 141.47289 121.492992) (width 0.5) (layer "F.Cu") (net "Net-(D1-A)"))
 (segment (start 141.47289 120.24093) (end 141.730743 119.983077) (width 0.5) (layer "F.Cu") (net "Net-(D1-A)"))
 (segment (start 141.47289 121.492992) (end 141.47289 120.24093) (width 0.5) (layer "F.Cu") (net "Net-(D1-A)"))
 (segment (start 147.19 131.5) (end 147.19 127.210102) (width 0.5) (layer "F.Cu") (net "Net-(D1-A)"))
 (segment (start 160.99 120.49) (end 165 124.5) (width 0.5) (layer "B.Cu") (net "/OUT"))
 (segment (start 165 124.5) (end 165 126.56) (width 0.5) (layer "B.Cu") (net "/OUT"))
 (segment (start 156 120.49) (end 160.99 120.49) (width 0.5) (layer "B.Cu") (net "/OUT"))
 (segment (start 165 126.56) (end 162.04 129.52) (width 0.5) (layer "B.Cu") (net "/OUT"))
 (segment (start 160.06 131.5) (end 162.04 129.52) (width 0.5) (layer "B.Cu") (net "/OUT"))
 (segment (start 154.81 131.5) (end 160.06 131.5) (width 0.5) (layer "B.Cu") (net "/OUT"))
 (segment (start 153 119) (end 153 123.73) (width 0.5) (layer "F.Cu") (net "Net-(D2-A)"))
 (segment (start 140.677154 126.42482) (end 140.4193 126.682674) (width 0.5) (layer "F.Cu") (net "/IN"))
 (segment (start 140.4193 126.682674) (end 139.16724 126.682674) (width 0.5) (layer "F.Cu") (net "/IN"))
 (segment (start 127 129.51) (end 127.01 129.51) (width 0.2) (layer "F.Cu") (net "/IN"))
 (segment (start 136.22 123.735434) (end 136.22 120.5) (width 0.5) (layer "F.Cu") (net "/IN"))
 (segment (start 127.01 129.51) (end 127.5 130) (width 0.2) (layer "F.Cu") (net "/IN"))
 (segment (start 139.16724 126.682674) (end 136.22 123.735434) (width 0.5) (layer "F.Cu") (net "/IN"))
 (segment (start 122.3 121.8) (end 122.3 124.81) (width 0.5) (layer "B.Cu") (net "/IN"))
 (segment (start 136.22 120.5) (end 136.22 122.75) (width 0.5) (layer "B.Cu") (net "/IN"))
 (segment (start 122.3 124.81) (end 127 129.51) (width 0.5) (layer "B.Cu") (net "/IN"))
 (segment (start 121 120.5) (end 122.3 121.8) (width 0.5) (layer "B.Cu") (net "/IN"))
 (segment (start 137.72 119) (end 136.22 120.5) (width 0.5) (layer "B.Cu") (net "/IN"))
 (segment (start 129.46 129.51) (end 127 129.51) (width 0.5) (layer "B.Cu") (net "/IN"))
 (segment (start 145.38 119) (end 137.72 119) (width 0.5) (layer "B.Cu") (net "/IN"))
 (segment (start 136.22 122.75) (end 129.46 129.51) (width 0.5) (layer "B.Cu") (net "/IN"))
 (segment (start 142.628769 120.881103) (end 142.886622 120.62325) (width 0.5) (layer "F.Cu") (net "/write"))
 (segment (start 142.886622 120.62325) (end 142.886622 119.371188) (width 0.5) (layer "F.Cu") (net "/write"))
 (segment (start 142.886622 119.371188) (end 141.475434 117.96) (width 0.5) (layer "F.Cu") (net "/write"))
 (segment (start 141.475434 117.96) (end 125 117.96) (width 0.5) (layer "F.Cu") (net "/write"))
 (segment (start 128.6 120.5) (end 128.6 122.33) (width 0.5) (layer "F.Cu") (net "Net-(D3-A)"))
 (segment (start 128.6 122.33) (end 130 123.73) (width 0.5) (layer "F.Cu") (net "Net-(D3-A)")))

